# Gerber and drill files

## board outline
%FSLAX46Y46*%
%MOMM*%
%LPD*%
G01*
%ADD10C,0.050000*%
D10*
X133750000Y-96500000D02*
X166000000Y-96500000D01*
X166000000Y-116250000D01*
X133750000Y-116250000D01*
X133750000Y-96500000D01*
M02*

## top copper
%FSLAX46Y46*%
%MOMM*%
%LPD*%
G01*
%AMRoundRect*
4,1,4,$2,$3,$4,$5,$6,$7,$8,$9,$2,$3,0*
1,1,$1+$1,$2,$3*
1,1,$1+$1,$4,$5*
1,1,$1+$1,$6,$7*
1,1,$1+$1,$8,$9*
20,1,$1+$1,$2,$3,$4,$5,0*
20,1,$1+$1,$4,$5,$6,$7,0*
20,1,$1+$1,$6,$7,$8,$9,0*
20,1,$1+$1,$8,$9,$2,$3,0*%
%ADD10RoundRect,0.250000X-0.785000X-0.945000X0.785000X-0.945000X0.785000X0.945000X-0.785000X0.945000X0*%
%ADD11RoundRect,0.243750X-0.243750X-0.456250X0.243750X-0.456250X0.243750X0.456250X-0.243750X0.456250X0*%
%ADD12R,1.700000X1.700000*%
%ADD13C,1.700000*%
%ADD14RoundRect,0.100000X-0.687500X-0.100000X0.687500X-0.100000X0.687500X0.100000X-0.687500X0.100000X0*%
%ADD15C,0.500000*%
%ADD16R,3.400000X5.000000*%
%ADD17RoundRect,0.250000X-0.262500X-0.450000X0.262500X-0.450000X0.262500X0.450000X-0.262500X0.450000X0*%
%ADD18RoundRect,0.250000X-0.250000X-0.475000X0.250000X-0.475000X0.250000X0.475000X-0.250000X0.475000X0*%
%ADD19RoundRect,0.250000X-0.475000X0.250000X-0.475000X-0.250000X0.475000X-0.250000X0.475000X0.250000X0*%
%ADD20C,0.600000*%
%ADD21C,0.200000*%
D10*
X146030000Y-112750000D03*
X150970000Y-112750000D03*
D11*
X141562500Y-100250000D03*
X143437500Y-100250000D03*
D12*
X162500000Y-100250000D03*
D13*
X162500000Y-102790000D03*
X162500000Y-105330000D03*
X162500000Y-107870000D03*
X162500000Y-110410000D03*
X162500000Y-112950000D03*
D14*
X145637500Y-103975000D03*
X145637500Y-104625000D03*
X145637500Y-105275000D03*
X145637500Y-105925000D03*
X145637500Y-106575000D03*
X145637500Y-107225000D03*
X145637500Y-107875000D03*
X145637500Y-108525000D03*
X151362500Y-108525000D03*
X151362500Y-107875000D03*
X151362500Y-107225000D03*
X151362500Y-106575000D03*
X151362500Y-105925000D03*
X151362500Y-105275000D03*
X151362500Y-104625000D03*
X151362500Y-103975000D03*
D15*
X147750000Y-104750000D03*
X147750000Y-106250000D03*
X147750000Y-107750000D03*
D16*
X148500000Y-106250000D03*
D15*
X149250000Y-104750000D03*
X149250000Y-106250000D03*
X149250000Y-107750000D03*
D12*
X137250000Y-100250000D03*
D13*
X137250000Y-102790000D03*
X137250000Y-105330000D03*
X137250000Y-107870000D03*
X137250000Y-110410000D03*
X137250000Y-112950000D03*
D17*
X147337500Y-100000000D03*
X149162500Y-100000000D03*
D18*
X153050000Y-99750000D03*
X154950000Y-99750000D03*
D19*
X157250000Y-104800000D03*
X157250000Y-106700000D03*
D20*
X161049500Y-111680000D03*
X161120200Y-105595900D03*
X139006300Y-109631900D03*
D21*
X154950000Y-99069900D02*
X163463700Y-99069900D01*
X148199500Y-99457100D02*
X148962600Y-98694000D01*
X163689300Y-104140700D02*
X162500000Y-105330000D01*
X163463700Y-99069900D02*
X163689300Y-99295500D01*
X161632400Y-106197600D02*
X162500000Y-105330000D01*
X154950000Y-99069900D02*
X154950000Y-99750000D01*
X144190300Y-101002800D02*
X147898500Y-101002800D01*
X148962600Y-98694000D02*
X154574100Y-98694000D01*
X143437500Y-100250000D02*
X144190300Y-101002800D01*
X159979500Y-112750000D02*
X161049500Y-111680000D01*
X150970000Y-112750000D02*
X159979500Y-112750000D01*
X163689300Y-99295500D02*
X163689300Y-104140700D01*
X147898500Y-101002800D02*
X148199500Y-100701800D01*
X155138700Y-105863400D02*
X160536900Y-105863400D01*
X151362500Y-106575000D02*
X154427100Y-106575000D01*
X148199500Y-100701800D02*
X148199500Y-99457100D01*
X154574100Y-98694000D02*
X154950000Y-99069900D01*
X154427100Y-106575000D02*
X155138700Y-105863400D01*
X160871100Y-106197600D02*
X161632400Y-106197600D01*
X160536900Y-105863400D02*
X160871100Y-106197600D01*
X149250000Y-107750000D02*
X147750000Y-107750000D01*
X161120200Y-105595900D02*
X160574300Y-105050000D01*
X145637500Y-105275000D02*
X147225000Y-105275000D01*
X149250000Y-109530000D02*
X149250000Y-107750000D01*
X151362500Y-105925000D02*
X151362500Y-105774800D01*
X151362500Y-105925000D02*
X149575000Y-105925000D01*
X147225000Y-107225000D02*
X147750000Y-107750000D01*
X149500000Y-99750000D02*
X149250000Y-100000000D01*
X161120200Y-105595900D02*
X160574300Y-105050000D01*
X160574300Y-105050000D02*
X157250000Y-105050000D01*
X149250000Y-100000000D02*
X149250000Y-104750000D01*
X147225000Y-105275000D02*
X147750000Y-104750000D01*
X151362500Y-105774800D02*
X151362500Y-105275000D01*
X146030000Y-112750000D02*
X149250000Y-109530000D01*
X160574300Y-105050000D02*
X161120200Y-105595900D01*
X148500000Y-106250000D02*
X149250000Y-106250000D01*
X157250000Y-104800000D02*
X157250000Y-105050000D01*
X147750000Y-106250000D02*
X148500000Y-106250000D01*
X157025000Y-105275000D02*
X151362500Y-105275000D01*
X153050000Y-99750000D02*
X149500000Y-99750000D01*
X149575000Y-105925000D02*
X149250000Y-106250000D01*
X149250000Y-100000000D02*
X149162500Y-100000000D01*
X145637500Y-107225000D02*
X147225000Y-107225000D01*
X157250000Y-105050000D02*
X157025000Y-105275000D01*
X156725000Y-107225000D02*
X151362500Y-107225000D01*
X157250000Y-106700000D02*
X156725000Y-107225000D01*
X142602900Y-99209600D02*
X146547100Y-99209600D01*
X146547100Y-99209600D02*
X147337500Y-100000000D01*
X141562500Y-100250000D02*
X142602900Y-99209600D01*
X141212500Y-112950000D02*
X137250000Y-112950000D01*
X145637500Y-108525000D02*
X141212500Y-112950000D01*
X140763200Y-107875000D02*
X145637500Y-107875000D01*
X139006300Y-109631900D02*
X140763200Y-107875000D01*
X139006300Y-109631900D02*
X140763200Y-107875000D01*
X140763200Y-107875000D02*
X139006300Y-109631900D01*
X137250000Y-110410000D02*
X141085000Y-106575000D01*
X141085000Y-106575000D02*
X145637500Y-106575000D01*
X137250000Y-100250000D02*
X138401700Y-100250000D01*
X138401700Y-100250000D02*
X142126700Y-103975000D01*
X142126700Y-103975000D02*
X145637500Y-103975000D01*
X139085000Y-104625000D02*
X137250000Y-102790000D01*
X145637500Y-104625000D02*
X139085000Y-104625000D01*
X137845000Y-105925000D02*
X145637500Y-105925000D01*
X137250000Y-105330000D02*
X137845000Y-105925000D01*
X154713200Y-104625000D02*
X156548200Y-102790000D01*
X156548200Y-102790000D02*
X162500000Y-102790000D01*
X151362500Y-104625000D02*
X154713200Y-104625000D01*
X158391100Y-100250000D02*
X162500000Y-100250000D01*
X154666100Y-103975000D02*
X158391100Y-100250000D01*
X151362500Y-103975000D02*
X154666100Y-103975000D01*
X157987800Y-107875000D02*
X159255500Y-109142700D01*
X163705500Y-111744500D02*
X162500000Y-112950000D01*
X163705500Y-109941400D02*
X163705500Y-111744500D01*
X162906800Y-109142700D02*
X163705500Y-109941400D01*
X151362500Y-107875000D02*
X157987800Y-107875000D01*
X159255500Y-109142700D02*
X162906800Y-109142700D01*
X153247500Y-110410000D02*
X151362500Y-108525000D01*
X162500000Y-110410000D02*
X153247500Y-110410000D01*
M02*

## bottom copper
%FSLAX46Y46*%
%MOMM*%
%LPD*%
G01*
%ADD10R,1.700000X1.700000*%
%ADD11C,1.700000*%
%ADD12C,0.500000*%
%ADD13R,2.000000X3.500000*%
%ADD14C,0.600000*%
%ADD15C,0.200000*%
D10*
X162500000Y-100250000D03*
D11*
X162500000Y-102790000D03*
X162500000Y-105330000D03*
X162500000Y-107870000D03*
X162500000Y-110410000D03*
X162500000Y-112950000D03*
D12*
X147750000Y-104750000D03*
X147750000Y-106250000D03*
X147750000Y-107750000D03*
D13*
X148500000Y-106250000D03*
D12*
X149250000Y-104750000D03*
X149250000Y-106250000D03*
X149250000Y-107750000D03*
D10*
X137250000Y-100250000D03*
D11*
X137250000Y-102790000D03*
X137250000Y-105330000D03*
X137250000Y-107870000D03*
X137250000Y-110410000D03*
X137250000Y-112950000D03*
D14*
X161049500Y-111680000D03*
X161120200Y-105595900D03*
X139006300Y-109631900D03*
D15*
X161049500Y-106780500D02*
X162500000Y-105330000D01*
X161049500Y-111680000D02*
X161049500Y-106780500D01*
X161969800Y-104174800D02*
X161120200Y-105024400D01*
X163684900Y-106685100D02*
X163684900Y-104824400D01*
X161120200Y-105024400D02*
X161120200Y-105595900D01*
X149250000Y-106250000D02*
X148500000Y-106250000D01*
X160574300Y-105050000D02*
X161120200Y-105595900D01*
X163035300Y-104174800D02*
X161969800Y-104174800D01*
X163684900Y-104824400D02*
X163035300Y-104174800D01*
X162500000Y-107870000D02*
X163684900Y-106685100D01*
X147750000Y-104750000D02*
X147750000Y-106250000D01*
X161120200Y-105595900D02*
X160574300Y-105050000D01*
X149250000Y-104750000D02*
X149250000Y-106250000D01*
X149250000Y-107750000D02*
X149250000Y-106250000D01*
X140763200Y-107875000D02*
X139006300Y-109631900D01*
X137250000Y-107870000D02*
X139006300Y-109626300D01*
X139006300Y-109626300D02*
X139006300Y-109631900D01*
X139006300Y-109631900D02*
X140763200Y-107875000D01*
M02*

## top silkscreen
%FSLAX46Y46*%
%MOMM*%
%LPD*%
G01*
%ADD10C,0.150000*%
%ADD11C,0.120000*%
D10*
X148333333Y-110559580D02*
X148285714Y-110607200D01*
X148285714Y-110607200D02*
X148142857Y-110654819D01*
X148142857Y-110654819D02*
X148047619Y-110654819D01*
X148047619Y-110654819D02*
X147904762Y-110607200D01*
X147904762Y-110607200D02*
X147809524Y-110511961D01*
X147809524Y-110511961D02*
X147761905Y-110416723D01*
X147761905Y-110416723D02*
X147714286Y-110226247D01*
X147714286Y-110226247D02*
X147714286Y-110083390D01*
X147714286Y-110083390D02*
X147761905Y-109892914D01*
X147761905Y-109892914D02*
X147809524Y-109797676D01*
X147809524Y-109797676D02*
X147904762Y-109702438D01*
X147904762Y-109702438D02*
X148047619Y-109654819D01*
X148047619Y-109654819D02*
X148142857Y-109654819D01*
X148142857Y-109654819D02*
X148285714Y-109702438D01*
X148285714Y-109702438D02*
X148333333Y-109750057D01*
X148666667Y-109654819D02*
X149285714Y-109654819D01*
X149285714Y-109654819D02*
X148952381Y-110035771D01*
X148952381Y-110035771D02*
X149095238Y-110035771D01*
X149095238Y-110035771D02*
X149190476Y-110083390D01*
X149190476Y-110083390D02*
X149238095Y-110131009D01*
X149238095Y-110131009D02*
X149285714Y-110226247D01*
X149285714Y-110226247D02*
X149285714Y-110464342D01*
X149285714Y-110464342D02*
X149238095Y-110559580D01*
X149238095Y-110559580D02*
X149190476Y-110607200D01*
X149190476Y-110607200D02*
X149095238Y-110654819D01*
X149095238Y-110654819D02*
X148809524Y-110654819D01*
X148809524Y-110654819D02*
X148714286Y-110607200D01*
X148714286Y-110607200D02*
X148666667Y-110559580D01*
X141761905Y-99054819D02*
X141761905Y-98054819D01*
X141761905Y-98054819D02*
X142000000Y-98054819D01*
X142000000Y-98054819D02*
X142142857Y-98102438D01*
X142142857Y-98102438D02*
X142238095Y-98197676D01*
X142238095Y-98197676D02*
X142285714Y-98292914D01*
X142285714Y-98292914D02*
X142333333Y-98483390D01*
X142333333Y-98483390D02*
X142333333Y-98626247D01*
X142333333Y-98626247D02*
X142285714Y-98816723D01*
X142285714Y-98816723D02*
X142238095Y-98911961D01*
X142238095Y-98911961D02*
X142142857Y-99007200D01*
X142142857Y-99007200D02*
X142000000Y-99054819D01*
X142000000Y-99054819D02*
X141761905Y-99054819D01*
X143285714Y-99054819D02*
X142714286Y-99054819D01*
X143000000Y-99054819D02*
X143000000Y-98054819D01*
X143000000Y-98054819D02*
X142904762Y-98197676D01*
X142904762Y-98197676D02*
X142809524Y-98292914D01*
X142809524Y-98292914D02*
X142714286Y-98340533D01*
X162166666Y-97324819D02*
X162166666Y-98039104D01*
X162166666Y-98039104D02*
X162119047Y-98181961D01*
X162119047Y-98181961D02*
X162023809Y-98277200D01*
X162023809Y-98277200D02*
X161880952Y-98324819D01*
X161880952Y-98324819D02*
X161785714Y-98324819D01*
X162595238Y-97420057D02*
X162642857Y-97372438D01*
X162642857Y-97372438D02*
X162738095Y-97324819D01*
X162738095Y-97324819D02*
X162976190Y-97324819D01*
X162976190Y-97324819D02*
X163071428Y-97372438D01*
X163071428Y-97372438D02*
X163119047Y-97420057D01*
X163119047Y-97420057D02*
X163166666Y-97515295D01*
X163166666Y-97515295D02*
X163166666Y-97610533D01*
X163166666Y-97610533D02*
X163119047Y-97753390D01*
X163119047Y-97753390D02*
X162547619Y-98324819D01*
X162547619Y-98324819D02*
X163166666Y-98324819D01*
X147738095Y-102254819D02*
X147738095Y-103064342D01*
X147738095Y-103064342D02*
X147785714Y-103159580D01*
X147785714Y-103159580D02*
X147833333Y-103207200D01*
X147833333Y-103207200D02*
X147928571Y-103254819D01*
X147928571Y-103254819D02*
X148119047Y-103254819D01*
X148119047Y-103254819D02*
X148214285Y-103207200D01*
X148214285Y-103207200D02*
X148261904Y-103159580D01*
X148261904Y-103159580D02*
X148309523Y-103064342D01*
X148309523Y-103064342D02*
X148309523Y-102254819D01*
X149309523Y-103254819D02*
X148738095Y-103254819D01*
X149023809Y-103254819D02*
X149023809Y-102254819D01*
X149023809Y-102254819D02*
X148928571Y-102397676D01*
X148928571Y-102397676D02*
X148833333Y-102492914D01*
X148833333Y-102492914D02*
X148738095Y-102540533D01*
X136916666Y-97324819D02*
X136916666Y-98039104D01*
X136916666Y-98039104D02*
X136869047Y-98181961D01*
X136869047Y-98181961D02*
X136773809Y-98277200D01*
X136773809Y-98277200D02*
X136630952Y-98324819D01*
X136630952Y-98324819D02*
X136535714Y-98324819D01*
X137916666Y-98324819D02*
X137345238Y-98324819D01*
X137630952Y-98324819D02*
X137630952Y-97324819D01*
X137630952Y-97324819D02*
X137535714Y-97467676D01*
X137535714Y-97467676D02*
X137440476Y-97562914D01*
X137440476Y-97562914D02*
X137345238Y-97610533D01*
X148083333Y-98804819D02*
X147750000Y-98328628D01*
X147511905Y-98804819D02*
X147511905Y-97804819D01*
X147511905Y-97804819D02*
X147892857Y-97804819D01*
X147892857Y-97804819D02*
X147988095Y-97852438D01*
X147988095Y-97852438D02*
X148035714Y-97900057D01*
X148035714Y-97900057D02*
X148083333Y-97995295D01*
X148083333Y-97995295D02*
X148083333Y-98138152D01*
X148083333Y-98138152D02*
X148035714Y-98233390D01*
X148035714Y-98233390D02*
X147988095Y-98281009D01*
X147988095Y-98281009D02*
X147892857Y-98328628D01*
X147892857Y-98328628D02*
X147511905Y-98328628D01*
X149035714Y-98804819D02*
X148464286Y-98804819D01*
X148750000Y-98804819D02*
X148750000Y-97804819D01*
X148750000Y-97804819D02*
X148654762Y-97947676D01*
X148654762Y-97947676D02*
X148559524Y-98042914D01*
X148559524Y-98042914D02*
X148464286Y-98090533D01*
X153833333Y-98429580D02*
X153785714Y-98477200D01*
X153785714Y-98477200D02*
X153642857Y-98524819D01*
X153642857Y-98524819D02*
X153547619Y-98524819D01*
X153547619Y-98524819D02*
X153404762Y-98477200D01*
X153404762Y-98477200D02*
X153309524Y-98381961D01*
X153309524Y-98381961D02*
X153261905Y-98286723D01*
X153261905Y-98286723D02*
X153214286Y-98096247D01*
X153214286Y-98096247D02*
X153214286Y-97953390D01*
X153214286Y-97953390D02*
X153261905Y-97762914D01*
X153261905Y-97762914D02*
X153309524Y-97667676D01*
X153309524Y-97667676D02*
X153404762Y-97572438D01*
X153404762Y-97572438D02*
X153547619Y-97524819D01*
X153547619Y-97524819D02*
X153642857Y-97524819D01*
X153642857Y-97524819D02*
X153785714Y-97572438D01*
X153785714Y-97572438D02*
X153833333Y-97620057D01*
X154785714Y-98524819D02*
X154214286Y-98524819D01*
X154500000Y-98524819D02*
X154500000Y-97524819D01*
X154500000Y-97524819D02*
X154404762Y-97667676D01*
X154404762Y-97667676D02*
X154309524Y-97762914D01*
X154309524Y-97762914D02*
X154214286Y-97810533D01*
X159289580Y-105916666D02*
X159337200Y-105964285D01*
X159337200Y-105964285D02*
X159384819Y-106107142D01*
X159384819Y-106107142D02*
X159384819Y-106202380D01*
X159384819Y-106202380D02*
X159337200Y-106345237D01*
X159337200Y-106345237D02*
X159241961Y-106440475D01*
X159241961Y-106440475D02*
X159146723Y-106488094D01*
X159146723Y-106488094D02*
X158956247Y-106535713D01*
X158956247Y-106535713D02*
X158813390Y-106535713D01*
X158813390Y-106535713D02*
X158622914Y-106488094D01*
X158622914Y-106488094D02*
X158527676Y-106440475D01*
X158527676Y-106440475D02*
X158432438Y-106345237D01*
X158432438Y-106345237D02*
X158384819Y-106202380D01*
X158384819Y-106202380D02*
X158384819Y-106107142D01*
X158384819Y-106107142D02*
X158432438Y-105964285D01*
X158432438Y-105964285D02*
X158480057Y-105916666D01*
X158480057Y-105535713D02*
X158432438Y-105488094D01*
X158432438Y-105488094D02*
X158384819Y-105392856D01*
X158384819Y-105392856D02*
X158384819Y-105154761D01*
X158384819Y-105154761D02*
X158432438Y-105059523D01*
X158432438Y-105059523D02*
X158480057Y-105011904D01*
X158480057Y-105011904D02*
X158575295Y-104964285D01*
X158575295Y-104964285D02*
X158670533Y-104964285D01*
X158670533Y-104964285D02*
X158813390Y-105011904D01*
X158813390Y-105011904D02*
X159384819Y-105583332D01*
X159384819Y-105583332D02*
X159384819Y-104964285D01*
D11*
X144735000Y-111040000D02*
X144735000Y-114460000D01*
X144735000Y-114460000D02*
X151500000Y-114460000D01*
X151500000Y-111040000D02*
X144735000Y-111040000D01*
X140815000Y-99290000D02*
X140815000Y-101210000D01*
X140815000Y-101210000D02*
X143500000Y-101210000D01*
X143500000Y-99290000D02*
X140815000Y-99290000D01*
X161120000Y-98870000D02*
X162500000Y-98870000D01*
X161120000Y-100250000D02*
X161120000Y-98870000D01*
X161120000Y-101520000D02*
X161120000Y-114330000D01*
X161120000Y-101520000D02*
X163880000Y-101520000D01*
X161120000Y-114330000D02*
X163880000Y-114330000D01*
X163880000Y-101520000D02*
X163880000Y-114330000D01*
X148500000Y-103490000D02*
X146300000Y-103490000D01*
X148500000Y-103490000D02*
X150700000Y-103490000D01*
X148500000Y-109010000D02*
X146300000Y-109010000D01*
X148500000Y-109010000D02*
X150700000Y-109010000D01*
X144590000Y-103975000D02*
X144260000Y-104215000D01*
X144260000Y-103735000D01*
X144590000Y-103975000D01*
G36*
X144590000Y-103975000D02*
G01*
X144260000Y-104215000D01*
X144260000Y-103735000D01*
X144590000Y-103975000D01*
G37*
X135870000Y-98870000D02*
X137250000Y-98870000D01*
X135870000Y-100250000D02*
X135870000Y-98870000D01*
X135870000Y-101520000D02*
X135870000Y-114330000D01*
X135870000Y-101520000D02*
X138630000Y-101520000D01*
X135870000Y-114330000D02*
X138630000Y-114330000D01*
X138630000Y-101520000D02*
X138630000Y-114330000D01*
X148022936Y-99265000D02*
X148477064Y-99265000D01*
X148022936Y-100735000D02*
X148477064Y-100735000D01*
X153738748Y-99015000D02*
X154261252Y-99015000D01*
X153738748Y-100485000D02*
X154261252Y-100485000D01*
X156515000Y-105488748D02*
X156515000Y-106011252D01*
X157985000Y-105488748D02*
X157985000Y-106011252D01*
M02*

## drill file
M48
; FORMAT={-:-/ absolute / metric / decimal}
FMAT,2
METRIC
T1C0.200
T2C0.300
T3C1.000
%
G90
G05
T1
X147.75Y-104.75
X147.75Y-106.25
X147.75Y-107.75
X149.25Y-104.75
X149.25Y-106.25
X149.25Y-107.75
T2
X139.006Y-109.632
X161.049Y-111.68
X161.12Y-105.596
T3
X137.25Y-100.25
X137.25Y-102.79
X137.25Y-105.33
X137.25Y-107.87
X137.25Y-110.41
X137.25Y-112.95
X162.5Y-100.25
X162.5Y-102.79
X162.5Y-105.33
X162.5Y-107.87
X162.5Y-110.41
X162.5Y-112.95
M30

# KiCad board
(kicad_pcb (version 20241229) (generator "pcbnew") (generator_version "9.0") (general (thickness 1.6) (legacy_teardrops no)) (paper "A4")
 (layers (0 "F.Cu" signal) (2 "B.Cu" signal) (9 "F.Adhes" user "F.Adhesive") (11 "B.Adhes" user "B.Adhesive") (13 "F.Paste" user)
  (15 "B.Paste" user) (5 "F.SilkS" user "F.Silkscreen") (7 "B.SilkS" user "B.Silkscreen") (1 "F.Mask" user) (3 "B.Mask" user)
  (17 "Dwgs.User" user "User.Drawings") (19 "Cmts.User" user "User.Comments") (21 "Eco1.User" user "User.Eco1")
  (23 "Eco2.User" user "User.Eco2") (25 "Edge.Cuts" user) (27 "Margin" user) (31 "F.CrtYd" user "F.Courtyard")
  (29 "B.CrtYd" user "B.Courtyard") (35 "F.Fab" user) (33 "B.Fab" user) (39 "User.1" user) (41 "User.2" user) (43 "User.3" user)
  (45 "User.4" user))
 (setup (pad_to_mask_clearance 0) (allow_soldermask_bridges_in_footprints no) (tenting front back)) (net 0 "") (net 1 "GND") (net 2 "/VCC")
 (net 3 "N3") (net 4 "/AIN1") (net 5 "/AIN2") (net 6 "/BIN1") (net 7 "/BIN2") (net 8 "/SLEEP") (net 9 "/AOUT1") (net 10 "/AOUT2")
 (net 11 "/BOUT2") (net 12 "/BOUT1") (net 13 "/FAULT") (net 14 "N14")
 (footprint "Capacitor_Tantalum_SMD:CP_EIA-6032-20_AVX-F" (layer "F.Cu") (at 148.5 112.75)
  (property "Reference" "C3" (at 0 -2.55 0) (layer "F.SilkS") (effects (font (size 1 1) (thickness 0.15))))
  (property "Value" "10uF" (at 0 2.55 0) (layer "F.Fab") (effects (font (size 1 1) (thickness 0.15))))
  (fp_line (start -3.765 -1.71) (end -3.765 1.71) (stroke (width 0.12) (type solid)) (layer "F.SilkS"))
  (fp_line (start -3.765 1.71) (end 3 1.71) (stroke (width 0.12) (type solid)) (layer "F.SilkS"))
  (fp_line (start 3 -1.71) (end -3.765 -1.71) (stroke (width 0.12) (type solid)) (layer "F.SilkS"))
  (pad "1" smd roundrect (at -2.47 0) (size 2.07 2.39) (layers "F.Cu" "F.Mask" "F.Paste") (roundrect_rratio 0.120773) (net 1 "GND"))
  (pad "2" smd roundrect (at 2.47 0) (size 2.07 2.39) (layers "F.Cu" "F.Mask" "F.Paste") (roundrect_rratio 0.120773) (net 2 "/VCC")))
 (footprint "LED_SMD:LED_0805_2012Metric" (layer "F.Cu") (at 142.5 100.25)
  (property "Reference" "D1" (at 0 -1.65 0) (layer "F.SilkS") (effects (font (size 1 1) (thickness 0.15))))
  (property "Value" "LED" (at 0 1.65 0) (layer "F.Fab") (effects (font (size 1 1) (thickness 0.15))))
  (fp_line (start -1.685 -0.96) (end -1.685 0.96) (stroke (width 0.12) (type solid)) (layer "F.SilkS"))
  (fp_line (start -1.685 0.96) (end 1 0.96) (stroke (width 0.12) (type solid)) (layer "F.SilkS"))
  (fp_line (start 1 -0.96) (end -1.685 -0.96) (stroke (width 0.12) (type solid)) (layer "F.SilkS"))
  (pad "1" smd roundrect (at -0.9375 0) (size 0.975 1.4) (layers "F.Cu" "F.Mask" "F.Paste") (roundrect_rratio 0.25) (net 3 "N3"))
  (pad "2" smd roundrect (at 0.9375 0) (size 0.975 1.4) (layers "F.Cu" "F.Mask" "F.Paste") (roundrect_rratio 0.25) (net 2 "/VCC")))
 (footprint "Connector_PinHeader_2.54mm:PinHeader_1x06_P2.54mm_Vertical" (layer "F.Cu") (at 162.5 100.25)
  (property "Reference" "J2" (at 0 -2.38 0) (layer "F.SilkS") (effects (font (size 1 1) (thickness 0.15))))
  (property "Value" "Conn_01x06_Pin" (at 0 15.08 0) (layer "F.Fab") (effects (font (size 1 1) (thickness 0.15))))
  (fp_line (start -1.38 -1.38) (end 0 -1.38) (stroke (width 0.12) (type solid)) (layer "F.SilkS"))
  (fp_line (start -1.38 0) (end -1.38 -1.38) (stroke (width 0.12) (type solid)) (layer "F.SilkS"))
  (fp_line (start -1.38 1.27) (end -1.38 14.08) (stroke (width 0.12) (type solid)) (layer "F.SilkS"))
  (fp_line (start -1.38 1.27) (end 1.38 1.27) (stroke (width 0.12) (type solid)) (layer "F.SilkS"))
  (fp_line (start -1.38 14.08) (end 1.38 14.08) (stroke (width 0.12) (type solid)) (layer "F.SilkS"))
  (fp_line (start 1.38 1.27) (end 1.38 14.08) (stroke (width 0.12) (type solid)) (layer "F.SilkS"))
  (pad "1" thru_hole rect (at 0 0) (size 1.7 1.7) (drill 1) (layers "*.Cu" "*.Mask") (remove_unused_layers no) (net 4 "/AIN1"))
  (pad "2" thru_hole circle (at 0 2.54) (size 1.7 1.7) (drill 1) (layers "*.Cu" "*.Mask") (remove_unused_layers no) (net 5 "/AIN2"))
  (pad "3" thru_hole circle (at 0 5.08) (size 1.7 1.7) (drill 1) (layers "*.Cu" "*.Mask") (remove_unused_layers no) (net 2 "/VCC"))
  (pad "4" thru_hole circle (at 0 7.62) (size 1.7 1.7) (drill 1) (layers "*.Cu" "*.Mask") (remove_unused_layers no) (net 1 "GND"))
  (pad "5" thru_hole circle (at 0 10.16) (size 1.7 1.7) (drill 1) (layers "*.Cu" "*.Mask") (remove_unused_layers no) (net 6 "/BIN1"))
  (pad "6" thru_hole circle (at 0 12.7) (size 1.7 1.7) (drill 1) (layers "*.Cu" "*.Mask") (remove_unused_layers no) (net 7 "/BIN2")))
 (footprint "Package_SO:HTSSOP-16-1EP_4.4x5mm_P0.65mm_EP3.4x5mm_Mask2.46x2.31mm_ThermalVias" (layer "F.Cu") (at 148.5 106.25)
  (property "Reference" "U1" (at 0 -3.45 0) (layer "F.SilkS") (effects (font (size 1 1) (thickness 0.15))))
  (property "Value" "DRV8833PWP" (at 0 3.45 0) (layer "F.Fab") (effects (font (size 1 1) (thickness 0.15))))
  (fp_line (start 0 -2.76) (end -2.2 -2.76) (stroke (width 0.12) (type solid)) (layer "F.SilkS"))
  (fp_line (start 0 -2.76) (end 2.2 -2.76) (stroke (width 0.12) (type solid)) (layer "F.SilkS"))
  (fp_line (start 0 2.76) (end -2.2 2.76) (stroke (width 0.12) (type solid)) (layer "F.SilkS"))
  (fp_line (start 0 2.76) (end 2.2 2.76) (stroke (width 0.12) (type solid)) (layer "F.SilkS"))
  (fp_poly (pts (xy -3.91 -2.275) (xy -4.24 -2.035) (xy -4.24 -2.515)) (stroke (width 0.12) (type solid)) (fill yes) (layer "F.SilkS"))
  (pad "" smd roundrect (at 0 -0.58) (size 1.98 0.93) (layers "F.Paste") (roundrect_rratio 0.25))
  (pad "" smd rect (at 0 0) (size 2.46 2.31) (layers "F.Mask"))
  (pad "" smd roundrect (at 0 0.58) (size 1.98 0.93) (layers "F.Paste") (roundrect_rratio 0.25))
  (pad "1" smd roundrect (at -2.8625 -2.275) (size 1.575 0.4) (layers "F.Cu" "F.Mask" "F.Paste") (roundrect_rratio 0.25) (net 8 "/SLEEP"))
  (pad "2" smd roundrect (at -2.8625 -1.625) (size 1.575 0.4) (layers "F.Cu" "F.Mask" "F.Paste") (roundrect_rratio 0.25) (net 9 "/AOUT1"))
  (pad "3" smd roundrect (at -2.8625 -0.975) (size 1.575 0.4) (layers "F.Cu" "F.Mask" "F.Paste") (roundrect_rratio 0.25) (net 1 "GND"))
  (pad "4" smd roundrect (at -2.8625 -0.325) (size 1.575 0.4) (layers "F.Cu" "F.Mask" "F.Paste") (roundrect_rratio 0.25) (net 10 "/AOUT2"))
  (pad "5" smd roundrect (at -2.8625 0.325) (size 1.575 0.4) (layers "F.Cu" "F.Mask" "F.Paste") (roundrect_rratio 0.25) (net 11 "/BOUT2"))
  (pad "6" smd roundrect (at -2.8625 0.975) (size 1.575 0.4) (layers "F.Cu" "F.Mask" "F.Paste") (roundrect_rratio 0.25) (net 1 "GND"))
  (pad "7" smd roundrect (at -2.8625 1.625) (size 1.575 0.4) (layers "F.Cu" "F.Mask" "F.Paste") (roundrect_rratio 0.25) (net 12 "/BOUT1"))
  (pad "8" smd roundrect (at -2.8625 2.275) (size 1.575 0.4) (layers "F.Cu" "F.Mask" "F.Paste") (roundrect_rratio 0.25) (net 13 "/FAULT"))
  (pad "9" smd roundrect (at 2.8625 2.275) (size 1.575 0.4) (layers "F.Cu" "F.Mask" "F.Paste") (roundrect_rratio 0.25) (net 6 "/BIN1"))
  (pad "10" smd roundrect (at 2.8625 1.625) (size 1.575 0.4) (layers "F.Cu" "F.Mask" "F.Paste") (roundrect_rratio 0.25) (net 7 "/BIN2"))
  (pad "11" smd roundrect (at 2.8625 0.975) (size 1.575 0.4) (layers "F.Cu" "F.Mask" "F.Paste") (roundrect_rratio 0.25) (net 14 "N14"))
  (pad "12" smd roundrect (at 2.8625 0.325) (size 1.575 0.4) (layers "F.Cu" "F.Mask" "F.Paste") (roundrect_rratio 0.25) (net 2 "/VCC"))
  (pad "13" smd roundrect (at 2.8625 -0.325) (size 1.575 0.4) (layers "F.Cu" "F.Mask" "F.Paste") (roundrect_rratio 0.25) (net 1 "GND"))
  (pad "14" smd roundrect (at 2.8625 -0.975) (size 1.575 0.4) (layers "F.Cu" "F.Mask" "F.Paste") (roundrect_rratio 0.25) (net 1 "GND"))
  (pad "15" smd roundrect (at 2.8625 -1.625) (size 1.575 0.4) (layers "F.Cu" "F.Mask" "F.Paste") (roundrect_rratio 0.25) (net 5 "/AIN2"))
  (pad "16" smd roundrect (at 2.8625 -2.275) (size 1.575 0.4) (layers "F.Cu" "F.Mask" "F.Paste") (roundrect_rratio 0.25) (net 4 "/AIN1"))
  (pad "17" thru_hole circle (at -0.75 -1.5) (size 0.5 0.5) (drill 0.2) (layers "*.Cu") (remove_unused_layers no) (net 1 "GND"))
  (pad "17" thru_hole circle (at -0.75 0) (size 0.5 0.5) (drill 0.2) (layers "*.Cu") (remove_unused_layers no) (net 1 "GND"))
  (pad "17" thru_hole circle (at -0.75 1.5) (size 0.5 0.5) (drill 0.2) (layers "*.Cu") (remove_unused_layers no) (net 1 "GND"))
  (pad "17" smd rect (at 0 0) (size 2 3.5) (layers "B.Cu") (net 1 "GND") (zone_connect 2))
  (pad "17" smd rect (at 0 0) (size 3.4 5) (layers "F.Cu") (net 1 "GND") (zone_connect 2))
  (pad "17" thru_hole circle (at 0.75 -1.5) (size 0.5 0.5) (drill 0.2) (layers "*.Cu") (remove_unused_layers no) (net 1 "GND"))
  (pad "17" thru_hole circle (at 0.75 0) (size 0.5 0.5) (drill 0.2) (layers "*.Cu") (remove_unused_layers no) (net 1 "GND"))
  (pad "17" thru_hole circle (at 0.75 1.5) (size 0.5 0.5) (drill 0.2) (layers "*.Cu") (remove_unused_layers no) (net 1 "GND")))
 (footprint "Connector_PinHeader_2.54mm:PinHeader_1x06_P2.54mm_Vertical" (layer "F.Cu") (at 137.25 100.25)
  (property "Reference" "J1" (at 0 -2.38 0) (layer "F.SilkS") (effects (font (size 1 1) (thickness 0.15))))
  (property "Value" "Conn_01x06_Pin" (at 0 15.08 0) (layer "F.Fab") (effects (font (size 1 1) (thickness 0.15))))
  (fp_line (start -1.38 -1.38) (end 0 -1.38) (stroke (width 0.12) (type solid)) (layer "F.SilkS"))
  (fp_line (start -1.38 0) (end -1.38 -1.38) (stroke (width 0.12) (type solid)) (layer "F.SilkS"))
  (fp_line (start -1.38 1.27) (end -1.38 14.08) (stroke (width 0.12) (type solid)) (layer "F.SilkS"))
  (fp_line (start -1.38 1.27) (end 1.38 1.27) (stroke (width 0.12) (type solid)) (layer "F.SilkS"))
  (fp_line (start -1.38 14.08) (end 1.38 14.08) (stroke (width 0.12) (type solid)) (layer "F.SilkS"))
  (fp_line (start 1.38 1.27) (end 1.38 14.08) (stroke (width 0.12) (type solid)) (layer "F.SilkS"))
  (pad "1" thru_hole rect (at 0 0) (size 1.7 1.7) (drill 1) (layers "*.Cu" "*.Mask") (remove_unused_layers no) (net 8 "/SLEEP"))
  (pad "2" thru_hole circle (at 0 2.54) (size 1.7 1.7) (drill 1) (layers "*.Cu" "*.Mask") (remove_unused_layers no) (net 9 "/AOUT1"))
  (pad "3" thru_hole circle (at 0 5.08) (size 1.7 1.7) (drill 1) (layers "*.Cu" "*.Mask") (remove_unused_layers no) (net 10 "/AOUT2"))
  (pad "4" thru_hole circle (at 0 7.62) (size 1.7 1.7) (drill 1) (layers "*.Cu" "*.Mask") (remove_unused_layers no) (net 12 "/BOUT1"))
  (pad "5" thru_hole circle (at 0 10.16) (size 1.7 1.7) (drill 1) (layers "*.Cu" "*.Mask") (remove_unused_layers no) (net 11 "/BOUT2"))
  (pad "6" thru_hole circle (at 0 12.7) (size 1.7 1.7) (drill 1) (layers "*.Cu" "*.Mask") (remove_unused_layers no) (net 13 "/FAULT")))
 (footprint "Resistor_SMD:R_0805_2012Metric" (layer "F.Cu") (at 148.25 100)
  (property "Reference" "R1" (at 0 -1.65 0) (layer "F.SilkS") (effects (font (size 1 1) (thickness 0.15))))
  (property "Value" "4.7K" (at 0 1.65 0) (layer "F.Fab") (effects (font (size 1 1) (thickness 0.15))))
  (fp_line (start -0.227064 -0.735) (end 0.227064 -0.735) (stroke (width 0.12) (type solid)) (layer "F.SilkS"))
  (fp_line (start -0.227064 0.735) (end 0.227064 0.735) (stroke (width 0.12) (type solid)) (layer "F.SilkS"))
  (pad "1" smd roundrect (at -0.9125 0) (size 1.025 1.4) (layers "F.Cu" "F.Mask" "F.Paste") (roundrect_rratio 0.243902) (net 3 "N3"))
  (pad "2" smd roundrect (at 0.9125 0) (size 1.025 1.4) (layers "F.Cu" "F.Mask" "F.Paste") (roundrect_rratio 0.243902) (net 1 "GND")))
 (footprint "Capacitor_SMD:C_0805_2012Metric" (layer "F.Cu") (at 154 99.75)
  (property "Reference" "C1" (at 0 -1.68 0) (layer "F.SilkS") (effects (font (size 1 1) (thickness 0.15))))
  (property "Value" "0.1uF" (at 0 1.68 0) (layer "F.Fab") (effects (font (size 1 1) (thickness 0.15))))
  (fp_line (start -0.261252 -0.735) (end 0.261252 -0.735) (stroke (width 0.12) (type solid)) (layer "F.SilkS"))
  (fp_line (start -0.261252 0.735) (end 0.261252 0.735) (stroke (width 0.12) (type solid)) (layer "F.SilkS"))
  (pad "1" smd roundrect (at -0.95 0) (size 1 1.45) (layers "F.Cu" "F.Mask" "F.Paste") (roundrect_rratio 0.25) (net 1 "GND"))
  (pad "2" smd roundrect (at 0.95 0) (size 1 1.45) (layers "F.Cu" "F.Mask" "F.Paste") (roundrect_rratio 0.25) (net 2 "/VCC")))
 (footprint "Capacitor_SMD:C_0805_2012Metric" (layer "F.Cu") (at 157.25 105.75 -90)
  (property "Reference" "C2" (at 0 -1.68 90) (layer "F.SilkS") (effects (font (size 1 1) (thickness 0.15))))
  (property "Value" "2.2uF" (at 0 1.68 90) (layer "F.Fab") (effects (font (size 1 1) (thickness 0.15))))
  (fp_line (start -0.261252 0.735) (end 0.261252 0.735) (stroke (width 0.12) (type solid)) (layer "F.SilkS"))
  (fp_line (start -0.261252 -0.735) (end 0.261252 -0.735) (stroke (width 0.12) (type solid)) (layer "F.SilkS"))
  (pad "1" smd roundrect (at -0.95 0 270) (size 1 1.45) (layers "F.Cu" "F.Mask" "F.Paste") (roundrect_rratio 0.25) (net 1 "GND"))
  (pad "2" smd roundrect (at 0.95 0 270) (size 1 1.45) (layers "F.Cu" "F.Mask" "F.Paste") (roundrect_rratio 0.25) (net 14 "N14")))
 (gr_rect (start 133.75 96.5) (end 166 116.25) (stroke (width 0.05) (type default)) (fill no) (layer "Edge.Cuts"))
 (segment (start 154.95 99.0699) (end 163.4637 99.0699) (width 0.2) (layer "F.Cu") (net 2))
 (segment (start 148.1995 99.4571) (end 148.9626 98.694) (width 0.2) (layer "F.Cu") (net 2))
 (segment (start 163.6893 104.1407) (end 162.5 105.33) (width 0.2) (layer "F.Cu") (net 2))
 (segment (start 163.4637 99.0699) (end 163.6893 99.2955) (width 0.2) (layer "F.Cu") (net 2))
 (segment (start 161.6324 106.1976) (end 162.5 105.33) (width 0.2) (layer "F.Cu") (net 2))
 (segment (start 154.95 99.0699) (end 154.95 99.75) (width 0.2) (layer "F.Cu") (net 2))
 (segment (start 144.1903 101.0028) (end 147.8985 101.0028) (width 0.2) (layer "F.Cu") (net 2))
 (segment (start 148.9626 98.694) (end 154.5741 98.694) (width 0.2) (layer "F.Cu") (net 2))
 (segment (start 143.4375 100.25) (end 144.1903 101.0028) (width 0.2) (layer "F.Cu") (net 2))
 (segment (start 159.9795 112.75) (end 161.0495 111.68) (width 0.2) (layer "F.Cu") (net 2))
 (segment (start 150.97 112.75) (end 159.9795 112.75) (width 0.2) (layer "F.Cu") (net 2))
 (segment (start 163.6893 99.2955) (end 163.6893 104.1407) (width 0.2) (layer "F.Cu") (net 2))
 (segment (start 147.8985 101.0028) (end 148.1995 100.7018) (width 0.2) (layer "F.Cu") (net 2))
 (segment (start 155.1387 105.8634) (end 160.5369 105.8634) (width 0.2) (layer "F.Cu") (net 2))
 (segment (start 151.3625 106.575) (end 154.4271 106.575) (width 0.2) (layer "F.Cu") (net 2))
 (segment (start 148.1995 100.7018) (end 148.1995 99.4571) (width 0.2) (layer "F.Cu") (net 2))
 (segment (start 154.5741 98.694) (end 154.95 99.0699) (width 0.2) (layer "F.Cu") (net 2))
 (segment (start 154.4271 106.575) (end 155.1387 105.8634) (width 0.2) (layer "F.Cu") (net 2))
 (segment (start 160.8711 106.1976) (end 161.6324 106.1976) (width 0.2) (layer "F.Cu") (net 2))
 (segment (start 160.5369 105.8634) (end 160.8711 106.1976) (width 0.2) (layer "F.Cu") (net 2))
 (via (at 161.0495 111.68) (size 0.6) (drill 0.3) (layers "F.Cu" "B.Cu") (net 2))
 (segment (start 161.0495 106.7805) (end 162.5 105.33) (width 0.2) (layer "B.Cu") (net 2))
 (segment (start 161.0495 111.68) (end 161.0495 106.7805) (width 0.2) (layer "B.Cu") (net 2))
 (segment (start 149.25 107.75) (end 147.75 107.75) (width 0.2) (layer "F.Cu") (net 1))
 (segment (start 161.1202 105.5959) (end 160.5743 105.05) (width 0.2) (layer "F.Cu") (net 1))
 (segment (start 145.6375 105.275) (end 147.225 105.275) (width 0.2) (layer "F.Cu") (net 1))
 (segment (start 149.25 109.53) (end 149.25 107.75) (width 0.2) (layer "F.Cu") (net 1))
 (segment (start 151.3625 105.925) (end 151.3625 105.7748) (width 0.2) (layer "F.Cu") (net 1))
 (segment (start 151.3625 105.925) (end 149.575 105.925) (width 0.2) (layer "F.Cu") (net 1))
 (segment (start 147.225 107.225) (end 147.75 107.75) (width 0.2) (layer "F.Cu") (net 1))
 (segment (start 149.5 99.75) (end 149.25 100) (width 0.2) (layer "F.Cu") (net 1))
 (segment (start 161.1202 105.5959) (end 160.5743 105.05) (width 0.2) (layer "F.Cu") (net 1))
 (segment (start 160.5743 105.05) (end 157.25 105.05) (width 0.2) (layer "F.Cu") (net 1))
 (segment (start 149.25 100) (end 149.25 104.75) (width 0.2) (layer "F.Cu") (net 1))
 (segment (start 147.225 105.275) (end 147.75 104.75) (width 0.2) (layer "F.Cu") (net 1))
 (segment (start 151.3625 105.7748) (end 151.3625 105.275) (width 0.2) (layer "F.Cu") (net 1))
 (segment (start 146.03 112.75) (end 149.25 109.53) (width 0.2) (layer "F.Cu") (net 1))
 (segment (start 160.5743 105.05) (end 161.1202 105.5959) (width 0.2) (layer "F.Cu") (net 1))
 (segment (start 148.5 106.25) (end 149.25 106.25) (width 0.2) (layer "F.Cu") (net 1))
 (segment (start 157.25 104.8) (end 157.25 105.05) (width 0.2) (layer "F.Cu") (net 1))
 (segment (start 147.75 106.25) (end 148.5 106.25) (width 0.2) (layer "F.Cu") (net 1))
 (segment (start 157.025 105.275) (end 151.3625 105.275) (width 0.2) (layer "F.Cu") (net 1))
 (segment (start 153.05 99.75) (end 149.5 99.75) (width 0.2) (layer "F.Cu") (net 1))
 (segment (start 149.575 105.925) (end 149.25 106.25) (width 0.2) (layer "F.Cu") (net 1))
 (segment (start 149.25 100) (end 149.1625 100) (width 0.2) (layer "F.Cu") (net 1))
 (segment (start 145.6375 107.225) (end 147.225 107.225) (width 0.2) (layer "F.Cu") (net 1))
 (segment (start 157.25 105.05) (end 157.025 105.275) (width 0.2) (layer "F.Cu") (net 1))
 (via (at 161.1202 105.5959) (size 0.6) (drill 0.3) (layers "F.Cu" "B.Cu") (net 1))
 (segment (start 161.9698 104.1748) (end 161.1202 105.0244) (width 0.2) (layer "B.Cu") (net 1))
 (segment (start 163.6849 106.6851) (end 163.6849 104.8244) (width 0.2) (layer "B.Cu") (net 1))
 (segment (start 161.1202 105.0244) (end 161.1202 105.5959) (width 0.2) (layer "B.Cu") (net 1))
 (segment (start 149.25 106.25) (end 148.5 106.25) (width 0.2) (layer "B.Cu") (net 1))
 (segment (start 160.5743 105.05) (end 161.1202 105.5959) (width 0.2) (layer "B.Cu") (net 1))
 (segment (start 163.0353 104.1748) (end 161.9698 104.1748) (width 0.2) (layer "B.Cu") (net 1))
 (segment (start 163.6849 104.8244) (end 163.0353 104.1748) (width 0.2) (layer "B.Cu") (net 1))
 (segment (start 162.5 107.87) (end 163.6849 106.6851) (width 0.2) (layer "B.Cu") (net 1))
 (segment (start 147.75 104.75) (end 147.75 106.25) (width 0.2) (layer "B.Cu") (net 1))
 (segment (start 161.1202 105.5959) (end 160.5743 105.05) (width 0.2) (layer "B.Cu") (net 1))
 (segment (start 149.25 104.75) (end 149.25 106.25) (width 0.2) (layer "B.Cu") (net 1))
 (segment (start 149.25 107.75) (end 149.25 106.25) (width 0.2) (layer "B.Cu") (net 1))
 (segment (start 156.725 107.225) (end 151.3625 107.225) (width 0.2) (layer "F.Cu") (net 14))
 (segment (start 157.25 106.7) (end 156.725 107.225) (width 0.2) (layer "F.Cu") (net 14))
 (segment (start 142.6029 99.2096) (end 146.5471 99.2096) (width 0.2) (layer "F.Cu") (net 3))
 (segment (start 146.5471 99.2096) (end 147.3375 100) (width 0.2) (layer "F.Cu") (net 3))
 (segment (start 141.5625 100.25) (end 142.6029 99.2096) (width 0.2) (layer "F.Cu") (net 3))
 (segment (start 141.2125 112.95) (end 137.25 112.95) (width 0.2) (layer "F.Cu") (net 13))
 (segment (start 145.6375 108.525) (end 141.2125 112.95) (width 0.2) (layer "F.Cu") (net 13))
 (segment (start 140.7632 107.875) (end 145.6375 107.875) (width 0.2) (layer "F.Cu") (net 12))
 (segment (start 139.0063 109.6319) (end 140.7632 107.875) (width 0.2) (layer "F.Cu") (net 12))
 (segment (start 139.0063 109.6319) (end 140.7632 107.875) (width 0.2) (layer "F.Cu") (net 12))
 (segment (start 140.7632 107.875) (end 139.0063 109.6319) (width 0.2) (layer "F.Cu") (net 12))
 (via (at 139.0063 109.6319) (size 0.6) (drill 0.3) (layers "F.Cu" "B.Cu") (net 12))
 (segment (start 140.7632 107.875) (end 139.0063 109.6319) (width 0.2) (layer "B.Cu") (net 12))
 (segment (start 137.25 107.87) (end 139.0063 109.6263) (width 0.2) (layer "B.Cu") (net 12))
 (segment (start 139.0063 109.6263) (end 139.0063 109.6319) (width 0.2) (layer "B.Cu") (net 12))
 (segment (start 139.0063 109.6319) (end 140.7632 107.875) (width 0.2) (layer "B.Cu") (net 12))
 (segment (start 137.25 110.41) (end 141.085 106.575) (width 0.2) (layer "F.Cu") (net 11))
 (segment (start 141.085 106.575) (end 145.6375 106.575) (width 0.2) (layer "F.Cu") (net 11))
 (segment (start 137.25 100.25) (end 138.4017 100.25) (width 0.2) (layer "F.Cu") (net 8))
 (segment (start 138.4017 100.25) (end 142.1267 103.975) (width 0.2) (layer "F.Cu") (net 8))
 (segment (start 142.1267 103.975) (end 145.6375 103.975) (width 0.2) (layer "F.Cu") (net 8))
 (segment (start 139.085 104.625) (end 137.25 102.79) (width 0.2) (layer "F.Cu") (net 9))
 (segment (start 145.6375 104.625) (end 139.085 104.625) (width 0.2) (layer "F.Cu") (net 9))
 (segment (start 137.845 105.925) (end 145.6375 105.925) (width 0.2) (layer "F.Cu") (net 10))
 (segment (start 137.25 105.33) (end 137.845 105.925) (width 0.2) (layer "F.Cu") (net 10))
 (segment (start 154.7132 104.625) (end 156.5482 102.79) (width 0.2) (layer "F.Cu") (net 5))
 (segment (start 156.5482 102.79) (end 162.5 102.79) (width 0.2) (layer "F.Cu") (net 5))
 (segment (start 151.3625 104.625) (end 154.7132 104.625) (width 0.2) (layer "F.Cu") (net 5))
 (segment (start 158.3911 100.25) (end 162.5 100.25) (width 0.2) (layer "F.Cu") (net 4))
 (segment (start 154.6661 103.975) (end 158.3911 100.25) (width 0.2) (layer "F.Cu") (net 4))
 (segment (start 151.3625 103.975) (end 154.6661 103.975) (width 0.2) (layer "F.Cu") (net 4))
 (segment (start 157.9878 107.875) (end 159.2555 109.1427) (width 0.2) (layer "F.Cu") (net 7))
 (segment (start 163.7055 111.7445) (end 162.5 112.95) (width 0.2) (layer "F.Cu") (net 7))
 (segment (start 163.7055 109.9414) (end 163.7055 111.7445) (width 0.2) (layer "F.Cu") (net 7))
 (segment (start 162.9068 109.1427) (end 163.7055 109.9414) (width 0.2) (layer "F.Cu") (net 7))
 (segment (start 151.3625 107.875) (end 157.9878 107.875) (width 0.2) (layer "F.Cu") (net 7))
 (segment (start 159.2555 109.1427) (end 162.9068 109.1427) (width 0.2) (layer "F.Cu") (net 7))
 (segment (start 153.2475 110.41) (end 151.3625 108.525) (width 0.2) (layer "F.Cu") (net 6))
 (segment (start 162.5 110.41) (end 153.2475 110.41) (width 0.2) (layer "F.Cu") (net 6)))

